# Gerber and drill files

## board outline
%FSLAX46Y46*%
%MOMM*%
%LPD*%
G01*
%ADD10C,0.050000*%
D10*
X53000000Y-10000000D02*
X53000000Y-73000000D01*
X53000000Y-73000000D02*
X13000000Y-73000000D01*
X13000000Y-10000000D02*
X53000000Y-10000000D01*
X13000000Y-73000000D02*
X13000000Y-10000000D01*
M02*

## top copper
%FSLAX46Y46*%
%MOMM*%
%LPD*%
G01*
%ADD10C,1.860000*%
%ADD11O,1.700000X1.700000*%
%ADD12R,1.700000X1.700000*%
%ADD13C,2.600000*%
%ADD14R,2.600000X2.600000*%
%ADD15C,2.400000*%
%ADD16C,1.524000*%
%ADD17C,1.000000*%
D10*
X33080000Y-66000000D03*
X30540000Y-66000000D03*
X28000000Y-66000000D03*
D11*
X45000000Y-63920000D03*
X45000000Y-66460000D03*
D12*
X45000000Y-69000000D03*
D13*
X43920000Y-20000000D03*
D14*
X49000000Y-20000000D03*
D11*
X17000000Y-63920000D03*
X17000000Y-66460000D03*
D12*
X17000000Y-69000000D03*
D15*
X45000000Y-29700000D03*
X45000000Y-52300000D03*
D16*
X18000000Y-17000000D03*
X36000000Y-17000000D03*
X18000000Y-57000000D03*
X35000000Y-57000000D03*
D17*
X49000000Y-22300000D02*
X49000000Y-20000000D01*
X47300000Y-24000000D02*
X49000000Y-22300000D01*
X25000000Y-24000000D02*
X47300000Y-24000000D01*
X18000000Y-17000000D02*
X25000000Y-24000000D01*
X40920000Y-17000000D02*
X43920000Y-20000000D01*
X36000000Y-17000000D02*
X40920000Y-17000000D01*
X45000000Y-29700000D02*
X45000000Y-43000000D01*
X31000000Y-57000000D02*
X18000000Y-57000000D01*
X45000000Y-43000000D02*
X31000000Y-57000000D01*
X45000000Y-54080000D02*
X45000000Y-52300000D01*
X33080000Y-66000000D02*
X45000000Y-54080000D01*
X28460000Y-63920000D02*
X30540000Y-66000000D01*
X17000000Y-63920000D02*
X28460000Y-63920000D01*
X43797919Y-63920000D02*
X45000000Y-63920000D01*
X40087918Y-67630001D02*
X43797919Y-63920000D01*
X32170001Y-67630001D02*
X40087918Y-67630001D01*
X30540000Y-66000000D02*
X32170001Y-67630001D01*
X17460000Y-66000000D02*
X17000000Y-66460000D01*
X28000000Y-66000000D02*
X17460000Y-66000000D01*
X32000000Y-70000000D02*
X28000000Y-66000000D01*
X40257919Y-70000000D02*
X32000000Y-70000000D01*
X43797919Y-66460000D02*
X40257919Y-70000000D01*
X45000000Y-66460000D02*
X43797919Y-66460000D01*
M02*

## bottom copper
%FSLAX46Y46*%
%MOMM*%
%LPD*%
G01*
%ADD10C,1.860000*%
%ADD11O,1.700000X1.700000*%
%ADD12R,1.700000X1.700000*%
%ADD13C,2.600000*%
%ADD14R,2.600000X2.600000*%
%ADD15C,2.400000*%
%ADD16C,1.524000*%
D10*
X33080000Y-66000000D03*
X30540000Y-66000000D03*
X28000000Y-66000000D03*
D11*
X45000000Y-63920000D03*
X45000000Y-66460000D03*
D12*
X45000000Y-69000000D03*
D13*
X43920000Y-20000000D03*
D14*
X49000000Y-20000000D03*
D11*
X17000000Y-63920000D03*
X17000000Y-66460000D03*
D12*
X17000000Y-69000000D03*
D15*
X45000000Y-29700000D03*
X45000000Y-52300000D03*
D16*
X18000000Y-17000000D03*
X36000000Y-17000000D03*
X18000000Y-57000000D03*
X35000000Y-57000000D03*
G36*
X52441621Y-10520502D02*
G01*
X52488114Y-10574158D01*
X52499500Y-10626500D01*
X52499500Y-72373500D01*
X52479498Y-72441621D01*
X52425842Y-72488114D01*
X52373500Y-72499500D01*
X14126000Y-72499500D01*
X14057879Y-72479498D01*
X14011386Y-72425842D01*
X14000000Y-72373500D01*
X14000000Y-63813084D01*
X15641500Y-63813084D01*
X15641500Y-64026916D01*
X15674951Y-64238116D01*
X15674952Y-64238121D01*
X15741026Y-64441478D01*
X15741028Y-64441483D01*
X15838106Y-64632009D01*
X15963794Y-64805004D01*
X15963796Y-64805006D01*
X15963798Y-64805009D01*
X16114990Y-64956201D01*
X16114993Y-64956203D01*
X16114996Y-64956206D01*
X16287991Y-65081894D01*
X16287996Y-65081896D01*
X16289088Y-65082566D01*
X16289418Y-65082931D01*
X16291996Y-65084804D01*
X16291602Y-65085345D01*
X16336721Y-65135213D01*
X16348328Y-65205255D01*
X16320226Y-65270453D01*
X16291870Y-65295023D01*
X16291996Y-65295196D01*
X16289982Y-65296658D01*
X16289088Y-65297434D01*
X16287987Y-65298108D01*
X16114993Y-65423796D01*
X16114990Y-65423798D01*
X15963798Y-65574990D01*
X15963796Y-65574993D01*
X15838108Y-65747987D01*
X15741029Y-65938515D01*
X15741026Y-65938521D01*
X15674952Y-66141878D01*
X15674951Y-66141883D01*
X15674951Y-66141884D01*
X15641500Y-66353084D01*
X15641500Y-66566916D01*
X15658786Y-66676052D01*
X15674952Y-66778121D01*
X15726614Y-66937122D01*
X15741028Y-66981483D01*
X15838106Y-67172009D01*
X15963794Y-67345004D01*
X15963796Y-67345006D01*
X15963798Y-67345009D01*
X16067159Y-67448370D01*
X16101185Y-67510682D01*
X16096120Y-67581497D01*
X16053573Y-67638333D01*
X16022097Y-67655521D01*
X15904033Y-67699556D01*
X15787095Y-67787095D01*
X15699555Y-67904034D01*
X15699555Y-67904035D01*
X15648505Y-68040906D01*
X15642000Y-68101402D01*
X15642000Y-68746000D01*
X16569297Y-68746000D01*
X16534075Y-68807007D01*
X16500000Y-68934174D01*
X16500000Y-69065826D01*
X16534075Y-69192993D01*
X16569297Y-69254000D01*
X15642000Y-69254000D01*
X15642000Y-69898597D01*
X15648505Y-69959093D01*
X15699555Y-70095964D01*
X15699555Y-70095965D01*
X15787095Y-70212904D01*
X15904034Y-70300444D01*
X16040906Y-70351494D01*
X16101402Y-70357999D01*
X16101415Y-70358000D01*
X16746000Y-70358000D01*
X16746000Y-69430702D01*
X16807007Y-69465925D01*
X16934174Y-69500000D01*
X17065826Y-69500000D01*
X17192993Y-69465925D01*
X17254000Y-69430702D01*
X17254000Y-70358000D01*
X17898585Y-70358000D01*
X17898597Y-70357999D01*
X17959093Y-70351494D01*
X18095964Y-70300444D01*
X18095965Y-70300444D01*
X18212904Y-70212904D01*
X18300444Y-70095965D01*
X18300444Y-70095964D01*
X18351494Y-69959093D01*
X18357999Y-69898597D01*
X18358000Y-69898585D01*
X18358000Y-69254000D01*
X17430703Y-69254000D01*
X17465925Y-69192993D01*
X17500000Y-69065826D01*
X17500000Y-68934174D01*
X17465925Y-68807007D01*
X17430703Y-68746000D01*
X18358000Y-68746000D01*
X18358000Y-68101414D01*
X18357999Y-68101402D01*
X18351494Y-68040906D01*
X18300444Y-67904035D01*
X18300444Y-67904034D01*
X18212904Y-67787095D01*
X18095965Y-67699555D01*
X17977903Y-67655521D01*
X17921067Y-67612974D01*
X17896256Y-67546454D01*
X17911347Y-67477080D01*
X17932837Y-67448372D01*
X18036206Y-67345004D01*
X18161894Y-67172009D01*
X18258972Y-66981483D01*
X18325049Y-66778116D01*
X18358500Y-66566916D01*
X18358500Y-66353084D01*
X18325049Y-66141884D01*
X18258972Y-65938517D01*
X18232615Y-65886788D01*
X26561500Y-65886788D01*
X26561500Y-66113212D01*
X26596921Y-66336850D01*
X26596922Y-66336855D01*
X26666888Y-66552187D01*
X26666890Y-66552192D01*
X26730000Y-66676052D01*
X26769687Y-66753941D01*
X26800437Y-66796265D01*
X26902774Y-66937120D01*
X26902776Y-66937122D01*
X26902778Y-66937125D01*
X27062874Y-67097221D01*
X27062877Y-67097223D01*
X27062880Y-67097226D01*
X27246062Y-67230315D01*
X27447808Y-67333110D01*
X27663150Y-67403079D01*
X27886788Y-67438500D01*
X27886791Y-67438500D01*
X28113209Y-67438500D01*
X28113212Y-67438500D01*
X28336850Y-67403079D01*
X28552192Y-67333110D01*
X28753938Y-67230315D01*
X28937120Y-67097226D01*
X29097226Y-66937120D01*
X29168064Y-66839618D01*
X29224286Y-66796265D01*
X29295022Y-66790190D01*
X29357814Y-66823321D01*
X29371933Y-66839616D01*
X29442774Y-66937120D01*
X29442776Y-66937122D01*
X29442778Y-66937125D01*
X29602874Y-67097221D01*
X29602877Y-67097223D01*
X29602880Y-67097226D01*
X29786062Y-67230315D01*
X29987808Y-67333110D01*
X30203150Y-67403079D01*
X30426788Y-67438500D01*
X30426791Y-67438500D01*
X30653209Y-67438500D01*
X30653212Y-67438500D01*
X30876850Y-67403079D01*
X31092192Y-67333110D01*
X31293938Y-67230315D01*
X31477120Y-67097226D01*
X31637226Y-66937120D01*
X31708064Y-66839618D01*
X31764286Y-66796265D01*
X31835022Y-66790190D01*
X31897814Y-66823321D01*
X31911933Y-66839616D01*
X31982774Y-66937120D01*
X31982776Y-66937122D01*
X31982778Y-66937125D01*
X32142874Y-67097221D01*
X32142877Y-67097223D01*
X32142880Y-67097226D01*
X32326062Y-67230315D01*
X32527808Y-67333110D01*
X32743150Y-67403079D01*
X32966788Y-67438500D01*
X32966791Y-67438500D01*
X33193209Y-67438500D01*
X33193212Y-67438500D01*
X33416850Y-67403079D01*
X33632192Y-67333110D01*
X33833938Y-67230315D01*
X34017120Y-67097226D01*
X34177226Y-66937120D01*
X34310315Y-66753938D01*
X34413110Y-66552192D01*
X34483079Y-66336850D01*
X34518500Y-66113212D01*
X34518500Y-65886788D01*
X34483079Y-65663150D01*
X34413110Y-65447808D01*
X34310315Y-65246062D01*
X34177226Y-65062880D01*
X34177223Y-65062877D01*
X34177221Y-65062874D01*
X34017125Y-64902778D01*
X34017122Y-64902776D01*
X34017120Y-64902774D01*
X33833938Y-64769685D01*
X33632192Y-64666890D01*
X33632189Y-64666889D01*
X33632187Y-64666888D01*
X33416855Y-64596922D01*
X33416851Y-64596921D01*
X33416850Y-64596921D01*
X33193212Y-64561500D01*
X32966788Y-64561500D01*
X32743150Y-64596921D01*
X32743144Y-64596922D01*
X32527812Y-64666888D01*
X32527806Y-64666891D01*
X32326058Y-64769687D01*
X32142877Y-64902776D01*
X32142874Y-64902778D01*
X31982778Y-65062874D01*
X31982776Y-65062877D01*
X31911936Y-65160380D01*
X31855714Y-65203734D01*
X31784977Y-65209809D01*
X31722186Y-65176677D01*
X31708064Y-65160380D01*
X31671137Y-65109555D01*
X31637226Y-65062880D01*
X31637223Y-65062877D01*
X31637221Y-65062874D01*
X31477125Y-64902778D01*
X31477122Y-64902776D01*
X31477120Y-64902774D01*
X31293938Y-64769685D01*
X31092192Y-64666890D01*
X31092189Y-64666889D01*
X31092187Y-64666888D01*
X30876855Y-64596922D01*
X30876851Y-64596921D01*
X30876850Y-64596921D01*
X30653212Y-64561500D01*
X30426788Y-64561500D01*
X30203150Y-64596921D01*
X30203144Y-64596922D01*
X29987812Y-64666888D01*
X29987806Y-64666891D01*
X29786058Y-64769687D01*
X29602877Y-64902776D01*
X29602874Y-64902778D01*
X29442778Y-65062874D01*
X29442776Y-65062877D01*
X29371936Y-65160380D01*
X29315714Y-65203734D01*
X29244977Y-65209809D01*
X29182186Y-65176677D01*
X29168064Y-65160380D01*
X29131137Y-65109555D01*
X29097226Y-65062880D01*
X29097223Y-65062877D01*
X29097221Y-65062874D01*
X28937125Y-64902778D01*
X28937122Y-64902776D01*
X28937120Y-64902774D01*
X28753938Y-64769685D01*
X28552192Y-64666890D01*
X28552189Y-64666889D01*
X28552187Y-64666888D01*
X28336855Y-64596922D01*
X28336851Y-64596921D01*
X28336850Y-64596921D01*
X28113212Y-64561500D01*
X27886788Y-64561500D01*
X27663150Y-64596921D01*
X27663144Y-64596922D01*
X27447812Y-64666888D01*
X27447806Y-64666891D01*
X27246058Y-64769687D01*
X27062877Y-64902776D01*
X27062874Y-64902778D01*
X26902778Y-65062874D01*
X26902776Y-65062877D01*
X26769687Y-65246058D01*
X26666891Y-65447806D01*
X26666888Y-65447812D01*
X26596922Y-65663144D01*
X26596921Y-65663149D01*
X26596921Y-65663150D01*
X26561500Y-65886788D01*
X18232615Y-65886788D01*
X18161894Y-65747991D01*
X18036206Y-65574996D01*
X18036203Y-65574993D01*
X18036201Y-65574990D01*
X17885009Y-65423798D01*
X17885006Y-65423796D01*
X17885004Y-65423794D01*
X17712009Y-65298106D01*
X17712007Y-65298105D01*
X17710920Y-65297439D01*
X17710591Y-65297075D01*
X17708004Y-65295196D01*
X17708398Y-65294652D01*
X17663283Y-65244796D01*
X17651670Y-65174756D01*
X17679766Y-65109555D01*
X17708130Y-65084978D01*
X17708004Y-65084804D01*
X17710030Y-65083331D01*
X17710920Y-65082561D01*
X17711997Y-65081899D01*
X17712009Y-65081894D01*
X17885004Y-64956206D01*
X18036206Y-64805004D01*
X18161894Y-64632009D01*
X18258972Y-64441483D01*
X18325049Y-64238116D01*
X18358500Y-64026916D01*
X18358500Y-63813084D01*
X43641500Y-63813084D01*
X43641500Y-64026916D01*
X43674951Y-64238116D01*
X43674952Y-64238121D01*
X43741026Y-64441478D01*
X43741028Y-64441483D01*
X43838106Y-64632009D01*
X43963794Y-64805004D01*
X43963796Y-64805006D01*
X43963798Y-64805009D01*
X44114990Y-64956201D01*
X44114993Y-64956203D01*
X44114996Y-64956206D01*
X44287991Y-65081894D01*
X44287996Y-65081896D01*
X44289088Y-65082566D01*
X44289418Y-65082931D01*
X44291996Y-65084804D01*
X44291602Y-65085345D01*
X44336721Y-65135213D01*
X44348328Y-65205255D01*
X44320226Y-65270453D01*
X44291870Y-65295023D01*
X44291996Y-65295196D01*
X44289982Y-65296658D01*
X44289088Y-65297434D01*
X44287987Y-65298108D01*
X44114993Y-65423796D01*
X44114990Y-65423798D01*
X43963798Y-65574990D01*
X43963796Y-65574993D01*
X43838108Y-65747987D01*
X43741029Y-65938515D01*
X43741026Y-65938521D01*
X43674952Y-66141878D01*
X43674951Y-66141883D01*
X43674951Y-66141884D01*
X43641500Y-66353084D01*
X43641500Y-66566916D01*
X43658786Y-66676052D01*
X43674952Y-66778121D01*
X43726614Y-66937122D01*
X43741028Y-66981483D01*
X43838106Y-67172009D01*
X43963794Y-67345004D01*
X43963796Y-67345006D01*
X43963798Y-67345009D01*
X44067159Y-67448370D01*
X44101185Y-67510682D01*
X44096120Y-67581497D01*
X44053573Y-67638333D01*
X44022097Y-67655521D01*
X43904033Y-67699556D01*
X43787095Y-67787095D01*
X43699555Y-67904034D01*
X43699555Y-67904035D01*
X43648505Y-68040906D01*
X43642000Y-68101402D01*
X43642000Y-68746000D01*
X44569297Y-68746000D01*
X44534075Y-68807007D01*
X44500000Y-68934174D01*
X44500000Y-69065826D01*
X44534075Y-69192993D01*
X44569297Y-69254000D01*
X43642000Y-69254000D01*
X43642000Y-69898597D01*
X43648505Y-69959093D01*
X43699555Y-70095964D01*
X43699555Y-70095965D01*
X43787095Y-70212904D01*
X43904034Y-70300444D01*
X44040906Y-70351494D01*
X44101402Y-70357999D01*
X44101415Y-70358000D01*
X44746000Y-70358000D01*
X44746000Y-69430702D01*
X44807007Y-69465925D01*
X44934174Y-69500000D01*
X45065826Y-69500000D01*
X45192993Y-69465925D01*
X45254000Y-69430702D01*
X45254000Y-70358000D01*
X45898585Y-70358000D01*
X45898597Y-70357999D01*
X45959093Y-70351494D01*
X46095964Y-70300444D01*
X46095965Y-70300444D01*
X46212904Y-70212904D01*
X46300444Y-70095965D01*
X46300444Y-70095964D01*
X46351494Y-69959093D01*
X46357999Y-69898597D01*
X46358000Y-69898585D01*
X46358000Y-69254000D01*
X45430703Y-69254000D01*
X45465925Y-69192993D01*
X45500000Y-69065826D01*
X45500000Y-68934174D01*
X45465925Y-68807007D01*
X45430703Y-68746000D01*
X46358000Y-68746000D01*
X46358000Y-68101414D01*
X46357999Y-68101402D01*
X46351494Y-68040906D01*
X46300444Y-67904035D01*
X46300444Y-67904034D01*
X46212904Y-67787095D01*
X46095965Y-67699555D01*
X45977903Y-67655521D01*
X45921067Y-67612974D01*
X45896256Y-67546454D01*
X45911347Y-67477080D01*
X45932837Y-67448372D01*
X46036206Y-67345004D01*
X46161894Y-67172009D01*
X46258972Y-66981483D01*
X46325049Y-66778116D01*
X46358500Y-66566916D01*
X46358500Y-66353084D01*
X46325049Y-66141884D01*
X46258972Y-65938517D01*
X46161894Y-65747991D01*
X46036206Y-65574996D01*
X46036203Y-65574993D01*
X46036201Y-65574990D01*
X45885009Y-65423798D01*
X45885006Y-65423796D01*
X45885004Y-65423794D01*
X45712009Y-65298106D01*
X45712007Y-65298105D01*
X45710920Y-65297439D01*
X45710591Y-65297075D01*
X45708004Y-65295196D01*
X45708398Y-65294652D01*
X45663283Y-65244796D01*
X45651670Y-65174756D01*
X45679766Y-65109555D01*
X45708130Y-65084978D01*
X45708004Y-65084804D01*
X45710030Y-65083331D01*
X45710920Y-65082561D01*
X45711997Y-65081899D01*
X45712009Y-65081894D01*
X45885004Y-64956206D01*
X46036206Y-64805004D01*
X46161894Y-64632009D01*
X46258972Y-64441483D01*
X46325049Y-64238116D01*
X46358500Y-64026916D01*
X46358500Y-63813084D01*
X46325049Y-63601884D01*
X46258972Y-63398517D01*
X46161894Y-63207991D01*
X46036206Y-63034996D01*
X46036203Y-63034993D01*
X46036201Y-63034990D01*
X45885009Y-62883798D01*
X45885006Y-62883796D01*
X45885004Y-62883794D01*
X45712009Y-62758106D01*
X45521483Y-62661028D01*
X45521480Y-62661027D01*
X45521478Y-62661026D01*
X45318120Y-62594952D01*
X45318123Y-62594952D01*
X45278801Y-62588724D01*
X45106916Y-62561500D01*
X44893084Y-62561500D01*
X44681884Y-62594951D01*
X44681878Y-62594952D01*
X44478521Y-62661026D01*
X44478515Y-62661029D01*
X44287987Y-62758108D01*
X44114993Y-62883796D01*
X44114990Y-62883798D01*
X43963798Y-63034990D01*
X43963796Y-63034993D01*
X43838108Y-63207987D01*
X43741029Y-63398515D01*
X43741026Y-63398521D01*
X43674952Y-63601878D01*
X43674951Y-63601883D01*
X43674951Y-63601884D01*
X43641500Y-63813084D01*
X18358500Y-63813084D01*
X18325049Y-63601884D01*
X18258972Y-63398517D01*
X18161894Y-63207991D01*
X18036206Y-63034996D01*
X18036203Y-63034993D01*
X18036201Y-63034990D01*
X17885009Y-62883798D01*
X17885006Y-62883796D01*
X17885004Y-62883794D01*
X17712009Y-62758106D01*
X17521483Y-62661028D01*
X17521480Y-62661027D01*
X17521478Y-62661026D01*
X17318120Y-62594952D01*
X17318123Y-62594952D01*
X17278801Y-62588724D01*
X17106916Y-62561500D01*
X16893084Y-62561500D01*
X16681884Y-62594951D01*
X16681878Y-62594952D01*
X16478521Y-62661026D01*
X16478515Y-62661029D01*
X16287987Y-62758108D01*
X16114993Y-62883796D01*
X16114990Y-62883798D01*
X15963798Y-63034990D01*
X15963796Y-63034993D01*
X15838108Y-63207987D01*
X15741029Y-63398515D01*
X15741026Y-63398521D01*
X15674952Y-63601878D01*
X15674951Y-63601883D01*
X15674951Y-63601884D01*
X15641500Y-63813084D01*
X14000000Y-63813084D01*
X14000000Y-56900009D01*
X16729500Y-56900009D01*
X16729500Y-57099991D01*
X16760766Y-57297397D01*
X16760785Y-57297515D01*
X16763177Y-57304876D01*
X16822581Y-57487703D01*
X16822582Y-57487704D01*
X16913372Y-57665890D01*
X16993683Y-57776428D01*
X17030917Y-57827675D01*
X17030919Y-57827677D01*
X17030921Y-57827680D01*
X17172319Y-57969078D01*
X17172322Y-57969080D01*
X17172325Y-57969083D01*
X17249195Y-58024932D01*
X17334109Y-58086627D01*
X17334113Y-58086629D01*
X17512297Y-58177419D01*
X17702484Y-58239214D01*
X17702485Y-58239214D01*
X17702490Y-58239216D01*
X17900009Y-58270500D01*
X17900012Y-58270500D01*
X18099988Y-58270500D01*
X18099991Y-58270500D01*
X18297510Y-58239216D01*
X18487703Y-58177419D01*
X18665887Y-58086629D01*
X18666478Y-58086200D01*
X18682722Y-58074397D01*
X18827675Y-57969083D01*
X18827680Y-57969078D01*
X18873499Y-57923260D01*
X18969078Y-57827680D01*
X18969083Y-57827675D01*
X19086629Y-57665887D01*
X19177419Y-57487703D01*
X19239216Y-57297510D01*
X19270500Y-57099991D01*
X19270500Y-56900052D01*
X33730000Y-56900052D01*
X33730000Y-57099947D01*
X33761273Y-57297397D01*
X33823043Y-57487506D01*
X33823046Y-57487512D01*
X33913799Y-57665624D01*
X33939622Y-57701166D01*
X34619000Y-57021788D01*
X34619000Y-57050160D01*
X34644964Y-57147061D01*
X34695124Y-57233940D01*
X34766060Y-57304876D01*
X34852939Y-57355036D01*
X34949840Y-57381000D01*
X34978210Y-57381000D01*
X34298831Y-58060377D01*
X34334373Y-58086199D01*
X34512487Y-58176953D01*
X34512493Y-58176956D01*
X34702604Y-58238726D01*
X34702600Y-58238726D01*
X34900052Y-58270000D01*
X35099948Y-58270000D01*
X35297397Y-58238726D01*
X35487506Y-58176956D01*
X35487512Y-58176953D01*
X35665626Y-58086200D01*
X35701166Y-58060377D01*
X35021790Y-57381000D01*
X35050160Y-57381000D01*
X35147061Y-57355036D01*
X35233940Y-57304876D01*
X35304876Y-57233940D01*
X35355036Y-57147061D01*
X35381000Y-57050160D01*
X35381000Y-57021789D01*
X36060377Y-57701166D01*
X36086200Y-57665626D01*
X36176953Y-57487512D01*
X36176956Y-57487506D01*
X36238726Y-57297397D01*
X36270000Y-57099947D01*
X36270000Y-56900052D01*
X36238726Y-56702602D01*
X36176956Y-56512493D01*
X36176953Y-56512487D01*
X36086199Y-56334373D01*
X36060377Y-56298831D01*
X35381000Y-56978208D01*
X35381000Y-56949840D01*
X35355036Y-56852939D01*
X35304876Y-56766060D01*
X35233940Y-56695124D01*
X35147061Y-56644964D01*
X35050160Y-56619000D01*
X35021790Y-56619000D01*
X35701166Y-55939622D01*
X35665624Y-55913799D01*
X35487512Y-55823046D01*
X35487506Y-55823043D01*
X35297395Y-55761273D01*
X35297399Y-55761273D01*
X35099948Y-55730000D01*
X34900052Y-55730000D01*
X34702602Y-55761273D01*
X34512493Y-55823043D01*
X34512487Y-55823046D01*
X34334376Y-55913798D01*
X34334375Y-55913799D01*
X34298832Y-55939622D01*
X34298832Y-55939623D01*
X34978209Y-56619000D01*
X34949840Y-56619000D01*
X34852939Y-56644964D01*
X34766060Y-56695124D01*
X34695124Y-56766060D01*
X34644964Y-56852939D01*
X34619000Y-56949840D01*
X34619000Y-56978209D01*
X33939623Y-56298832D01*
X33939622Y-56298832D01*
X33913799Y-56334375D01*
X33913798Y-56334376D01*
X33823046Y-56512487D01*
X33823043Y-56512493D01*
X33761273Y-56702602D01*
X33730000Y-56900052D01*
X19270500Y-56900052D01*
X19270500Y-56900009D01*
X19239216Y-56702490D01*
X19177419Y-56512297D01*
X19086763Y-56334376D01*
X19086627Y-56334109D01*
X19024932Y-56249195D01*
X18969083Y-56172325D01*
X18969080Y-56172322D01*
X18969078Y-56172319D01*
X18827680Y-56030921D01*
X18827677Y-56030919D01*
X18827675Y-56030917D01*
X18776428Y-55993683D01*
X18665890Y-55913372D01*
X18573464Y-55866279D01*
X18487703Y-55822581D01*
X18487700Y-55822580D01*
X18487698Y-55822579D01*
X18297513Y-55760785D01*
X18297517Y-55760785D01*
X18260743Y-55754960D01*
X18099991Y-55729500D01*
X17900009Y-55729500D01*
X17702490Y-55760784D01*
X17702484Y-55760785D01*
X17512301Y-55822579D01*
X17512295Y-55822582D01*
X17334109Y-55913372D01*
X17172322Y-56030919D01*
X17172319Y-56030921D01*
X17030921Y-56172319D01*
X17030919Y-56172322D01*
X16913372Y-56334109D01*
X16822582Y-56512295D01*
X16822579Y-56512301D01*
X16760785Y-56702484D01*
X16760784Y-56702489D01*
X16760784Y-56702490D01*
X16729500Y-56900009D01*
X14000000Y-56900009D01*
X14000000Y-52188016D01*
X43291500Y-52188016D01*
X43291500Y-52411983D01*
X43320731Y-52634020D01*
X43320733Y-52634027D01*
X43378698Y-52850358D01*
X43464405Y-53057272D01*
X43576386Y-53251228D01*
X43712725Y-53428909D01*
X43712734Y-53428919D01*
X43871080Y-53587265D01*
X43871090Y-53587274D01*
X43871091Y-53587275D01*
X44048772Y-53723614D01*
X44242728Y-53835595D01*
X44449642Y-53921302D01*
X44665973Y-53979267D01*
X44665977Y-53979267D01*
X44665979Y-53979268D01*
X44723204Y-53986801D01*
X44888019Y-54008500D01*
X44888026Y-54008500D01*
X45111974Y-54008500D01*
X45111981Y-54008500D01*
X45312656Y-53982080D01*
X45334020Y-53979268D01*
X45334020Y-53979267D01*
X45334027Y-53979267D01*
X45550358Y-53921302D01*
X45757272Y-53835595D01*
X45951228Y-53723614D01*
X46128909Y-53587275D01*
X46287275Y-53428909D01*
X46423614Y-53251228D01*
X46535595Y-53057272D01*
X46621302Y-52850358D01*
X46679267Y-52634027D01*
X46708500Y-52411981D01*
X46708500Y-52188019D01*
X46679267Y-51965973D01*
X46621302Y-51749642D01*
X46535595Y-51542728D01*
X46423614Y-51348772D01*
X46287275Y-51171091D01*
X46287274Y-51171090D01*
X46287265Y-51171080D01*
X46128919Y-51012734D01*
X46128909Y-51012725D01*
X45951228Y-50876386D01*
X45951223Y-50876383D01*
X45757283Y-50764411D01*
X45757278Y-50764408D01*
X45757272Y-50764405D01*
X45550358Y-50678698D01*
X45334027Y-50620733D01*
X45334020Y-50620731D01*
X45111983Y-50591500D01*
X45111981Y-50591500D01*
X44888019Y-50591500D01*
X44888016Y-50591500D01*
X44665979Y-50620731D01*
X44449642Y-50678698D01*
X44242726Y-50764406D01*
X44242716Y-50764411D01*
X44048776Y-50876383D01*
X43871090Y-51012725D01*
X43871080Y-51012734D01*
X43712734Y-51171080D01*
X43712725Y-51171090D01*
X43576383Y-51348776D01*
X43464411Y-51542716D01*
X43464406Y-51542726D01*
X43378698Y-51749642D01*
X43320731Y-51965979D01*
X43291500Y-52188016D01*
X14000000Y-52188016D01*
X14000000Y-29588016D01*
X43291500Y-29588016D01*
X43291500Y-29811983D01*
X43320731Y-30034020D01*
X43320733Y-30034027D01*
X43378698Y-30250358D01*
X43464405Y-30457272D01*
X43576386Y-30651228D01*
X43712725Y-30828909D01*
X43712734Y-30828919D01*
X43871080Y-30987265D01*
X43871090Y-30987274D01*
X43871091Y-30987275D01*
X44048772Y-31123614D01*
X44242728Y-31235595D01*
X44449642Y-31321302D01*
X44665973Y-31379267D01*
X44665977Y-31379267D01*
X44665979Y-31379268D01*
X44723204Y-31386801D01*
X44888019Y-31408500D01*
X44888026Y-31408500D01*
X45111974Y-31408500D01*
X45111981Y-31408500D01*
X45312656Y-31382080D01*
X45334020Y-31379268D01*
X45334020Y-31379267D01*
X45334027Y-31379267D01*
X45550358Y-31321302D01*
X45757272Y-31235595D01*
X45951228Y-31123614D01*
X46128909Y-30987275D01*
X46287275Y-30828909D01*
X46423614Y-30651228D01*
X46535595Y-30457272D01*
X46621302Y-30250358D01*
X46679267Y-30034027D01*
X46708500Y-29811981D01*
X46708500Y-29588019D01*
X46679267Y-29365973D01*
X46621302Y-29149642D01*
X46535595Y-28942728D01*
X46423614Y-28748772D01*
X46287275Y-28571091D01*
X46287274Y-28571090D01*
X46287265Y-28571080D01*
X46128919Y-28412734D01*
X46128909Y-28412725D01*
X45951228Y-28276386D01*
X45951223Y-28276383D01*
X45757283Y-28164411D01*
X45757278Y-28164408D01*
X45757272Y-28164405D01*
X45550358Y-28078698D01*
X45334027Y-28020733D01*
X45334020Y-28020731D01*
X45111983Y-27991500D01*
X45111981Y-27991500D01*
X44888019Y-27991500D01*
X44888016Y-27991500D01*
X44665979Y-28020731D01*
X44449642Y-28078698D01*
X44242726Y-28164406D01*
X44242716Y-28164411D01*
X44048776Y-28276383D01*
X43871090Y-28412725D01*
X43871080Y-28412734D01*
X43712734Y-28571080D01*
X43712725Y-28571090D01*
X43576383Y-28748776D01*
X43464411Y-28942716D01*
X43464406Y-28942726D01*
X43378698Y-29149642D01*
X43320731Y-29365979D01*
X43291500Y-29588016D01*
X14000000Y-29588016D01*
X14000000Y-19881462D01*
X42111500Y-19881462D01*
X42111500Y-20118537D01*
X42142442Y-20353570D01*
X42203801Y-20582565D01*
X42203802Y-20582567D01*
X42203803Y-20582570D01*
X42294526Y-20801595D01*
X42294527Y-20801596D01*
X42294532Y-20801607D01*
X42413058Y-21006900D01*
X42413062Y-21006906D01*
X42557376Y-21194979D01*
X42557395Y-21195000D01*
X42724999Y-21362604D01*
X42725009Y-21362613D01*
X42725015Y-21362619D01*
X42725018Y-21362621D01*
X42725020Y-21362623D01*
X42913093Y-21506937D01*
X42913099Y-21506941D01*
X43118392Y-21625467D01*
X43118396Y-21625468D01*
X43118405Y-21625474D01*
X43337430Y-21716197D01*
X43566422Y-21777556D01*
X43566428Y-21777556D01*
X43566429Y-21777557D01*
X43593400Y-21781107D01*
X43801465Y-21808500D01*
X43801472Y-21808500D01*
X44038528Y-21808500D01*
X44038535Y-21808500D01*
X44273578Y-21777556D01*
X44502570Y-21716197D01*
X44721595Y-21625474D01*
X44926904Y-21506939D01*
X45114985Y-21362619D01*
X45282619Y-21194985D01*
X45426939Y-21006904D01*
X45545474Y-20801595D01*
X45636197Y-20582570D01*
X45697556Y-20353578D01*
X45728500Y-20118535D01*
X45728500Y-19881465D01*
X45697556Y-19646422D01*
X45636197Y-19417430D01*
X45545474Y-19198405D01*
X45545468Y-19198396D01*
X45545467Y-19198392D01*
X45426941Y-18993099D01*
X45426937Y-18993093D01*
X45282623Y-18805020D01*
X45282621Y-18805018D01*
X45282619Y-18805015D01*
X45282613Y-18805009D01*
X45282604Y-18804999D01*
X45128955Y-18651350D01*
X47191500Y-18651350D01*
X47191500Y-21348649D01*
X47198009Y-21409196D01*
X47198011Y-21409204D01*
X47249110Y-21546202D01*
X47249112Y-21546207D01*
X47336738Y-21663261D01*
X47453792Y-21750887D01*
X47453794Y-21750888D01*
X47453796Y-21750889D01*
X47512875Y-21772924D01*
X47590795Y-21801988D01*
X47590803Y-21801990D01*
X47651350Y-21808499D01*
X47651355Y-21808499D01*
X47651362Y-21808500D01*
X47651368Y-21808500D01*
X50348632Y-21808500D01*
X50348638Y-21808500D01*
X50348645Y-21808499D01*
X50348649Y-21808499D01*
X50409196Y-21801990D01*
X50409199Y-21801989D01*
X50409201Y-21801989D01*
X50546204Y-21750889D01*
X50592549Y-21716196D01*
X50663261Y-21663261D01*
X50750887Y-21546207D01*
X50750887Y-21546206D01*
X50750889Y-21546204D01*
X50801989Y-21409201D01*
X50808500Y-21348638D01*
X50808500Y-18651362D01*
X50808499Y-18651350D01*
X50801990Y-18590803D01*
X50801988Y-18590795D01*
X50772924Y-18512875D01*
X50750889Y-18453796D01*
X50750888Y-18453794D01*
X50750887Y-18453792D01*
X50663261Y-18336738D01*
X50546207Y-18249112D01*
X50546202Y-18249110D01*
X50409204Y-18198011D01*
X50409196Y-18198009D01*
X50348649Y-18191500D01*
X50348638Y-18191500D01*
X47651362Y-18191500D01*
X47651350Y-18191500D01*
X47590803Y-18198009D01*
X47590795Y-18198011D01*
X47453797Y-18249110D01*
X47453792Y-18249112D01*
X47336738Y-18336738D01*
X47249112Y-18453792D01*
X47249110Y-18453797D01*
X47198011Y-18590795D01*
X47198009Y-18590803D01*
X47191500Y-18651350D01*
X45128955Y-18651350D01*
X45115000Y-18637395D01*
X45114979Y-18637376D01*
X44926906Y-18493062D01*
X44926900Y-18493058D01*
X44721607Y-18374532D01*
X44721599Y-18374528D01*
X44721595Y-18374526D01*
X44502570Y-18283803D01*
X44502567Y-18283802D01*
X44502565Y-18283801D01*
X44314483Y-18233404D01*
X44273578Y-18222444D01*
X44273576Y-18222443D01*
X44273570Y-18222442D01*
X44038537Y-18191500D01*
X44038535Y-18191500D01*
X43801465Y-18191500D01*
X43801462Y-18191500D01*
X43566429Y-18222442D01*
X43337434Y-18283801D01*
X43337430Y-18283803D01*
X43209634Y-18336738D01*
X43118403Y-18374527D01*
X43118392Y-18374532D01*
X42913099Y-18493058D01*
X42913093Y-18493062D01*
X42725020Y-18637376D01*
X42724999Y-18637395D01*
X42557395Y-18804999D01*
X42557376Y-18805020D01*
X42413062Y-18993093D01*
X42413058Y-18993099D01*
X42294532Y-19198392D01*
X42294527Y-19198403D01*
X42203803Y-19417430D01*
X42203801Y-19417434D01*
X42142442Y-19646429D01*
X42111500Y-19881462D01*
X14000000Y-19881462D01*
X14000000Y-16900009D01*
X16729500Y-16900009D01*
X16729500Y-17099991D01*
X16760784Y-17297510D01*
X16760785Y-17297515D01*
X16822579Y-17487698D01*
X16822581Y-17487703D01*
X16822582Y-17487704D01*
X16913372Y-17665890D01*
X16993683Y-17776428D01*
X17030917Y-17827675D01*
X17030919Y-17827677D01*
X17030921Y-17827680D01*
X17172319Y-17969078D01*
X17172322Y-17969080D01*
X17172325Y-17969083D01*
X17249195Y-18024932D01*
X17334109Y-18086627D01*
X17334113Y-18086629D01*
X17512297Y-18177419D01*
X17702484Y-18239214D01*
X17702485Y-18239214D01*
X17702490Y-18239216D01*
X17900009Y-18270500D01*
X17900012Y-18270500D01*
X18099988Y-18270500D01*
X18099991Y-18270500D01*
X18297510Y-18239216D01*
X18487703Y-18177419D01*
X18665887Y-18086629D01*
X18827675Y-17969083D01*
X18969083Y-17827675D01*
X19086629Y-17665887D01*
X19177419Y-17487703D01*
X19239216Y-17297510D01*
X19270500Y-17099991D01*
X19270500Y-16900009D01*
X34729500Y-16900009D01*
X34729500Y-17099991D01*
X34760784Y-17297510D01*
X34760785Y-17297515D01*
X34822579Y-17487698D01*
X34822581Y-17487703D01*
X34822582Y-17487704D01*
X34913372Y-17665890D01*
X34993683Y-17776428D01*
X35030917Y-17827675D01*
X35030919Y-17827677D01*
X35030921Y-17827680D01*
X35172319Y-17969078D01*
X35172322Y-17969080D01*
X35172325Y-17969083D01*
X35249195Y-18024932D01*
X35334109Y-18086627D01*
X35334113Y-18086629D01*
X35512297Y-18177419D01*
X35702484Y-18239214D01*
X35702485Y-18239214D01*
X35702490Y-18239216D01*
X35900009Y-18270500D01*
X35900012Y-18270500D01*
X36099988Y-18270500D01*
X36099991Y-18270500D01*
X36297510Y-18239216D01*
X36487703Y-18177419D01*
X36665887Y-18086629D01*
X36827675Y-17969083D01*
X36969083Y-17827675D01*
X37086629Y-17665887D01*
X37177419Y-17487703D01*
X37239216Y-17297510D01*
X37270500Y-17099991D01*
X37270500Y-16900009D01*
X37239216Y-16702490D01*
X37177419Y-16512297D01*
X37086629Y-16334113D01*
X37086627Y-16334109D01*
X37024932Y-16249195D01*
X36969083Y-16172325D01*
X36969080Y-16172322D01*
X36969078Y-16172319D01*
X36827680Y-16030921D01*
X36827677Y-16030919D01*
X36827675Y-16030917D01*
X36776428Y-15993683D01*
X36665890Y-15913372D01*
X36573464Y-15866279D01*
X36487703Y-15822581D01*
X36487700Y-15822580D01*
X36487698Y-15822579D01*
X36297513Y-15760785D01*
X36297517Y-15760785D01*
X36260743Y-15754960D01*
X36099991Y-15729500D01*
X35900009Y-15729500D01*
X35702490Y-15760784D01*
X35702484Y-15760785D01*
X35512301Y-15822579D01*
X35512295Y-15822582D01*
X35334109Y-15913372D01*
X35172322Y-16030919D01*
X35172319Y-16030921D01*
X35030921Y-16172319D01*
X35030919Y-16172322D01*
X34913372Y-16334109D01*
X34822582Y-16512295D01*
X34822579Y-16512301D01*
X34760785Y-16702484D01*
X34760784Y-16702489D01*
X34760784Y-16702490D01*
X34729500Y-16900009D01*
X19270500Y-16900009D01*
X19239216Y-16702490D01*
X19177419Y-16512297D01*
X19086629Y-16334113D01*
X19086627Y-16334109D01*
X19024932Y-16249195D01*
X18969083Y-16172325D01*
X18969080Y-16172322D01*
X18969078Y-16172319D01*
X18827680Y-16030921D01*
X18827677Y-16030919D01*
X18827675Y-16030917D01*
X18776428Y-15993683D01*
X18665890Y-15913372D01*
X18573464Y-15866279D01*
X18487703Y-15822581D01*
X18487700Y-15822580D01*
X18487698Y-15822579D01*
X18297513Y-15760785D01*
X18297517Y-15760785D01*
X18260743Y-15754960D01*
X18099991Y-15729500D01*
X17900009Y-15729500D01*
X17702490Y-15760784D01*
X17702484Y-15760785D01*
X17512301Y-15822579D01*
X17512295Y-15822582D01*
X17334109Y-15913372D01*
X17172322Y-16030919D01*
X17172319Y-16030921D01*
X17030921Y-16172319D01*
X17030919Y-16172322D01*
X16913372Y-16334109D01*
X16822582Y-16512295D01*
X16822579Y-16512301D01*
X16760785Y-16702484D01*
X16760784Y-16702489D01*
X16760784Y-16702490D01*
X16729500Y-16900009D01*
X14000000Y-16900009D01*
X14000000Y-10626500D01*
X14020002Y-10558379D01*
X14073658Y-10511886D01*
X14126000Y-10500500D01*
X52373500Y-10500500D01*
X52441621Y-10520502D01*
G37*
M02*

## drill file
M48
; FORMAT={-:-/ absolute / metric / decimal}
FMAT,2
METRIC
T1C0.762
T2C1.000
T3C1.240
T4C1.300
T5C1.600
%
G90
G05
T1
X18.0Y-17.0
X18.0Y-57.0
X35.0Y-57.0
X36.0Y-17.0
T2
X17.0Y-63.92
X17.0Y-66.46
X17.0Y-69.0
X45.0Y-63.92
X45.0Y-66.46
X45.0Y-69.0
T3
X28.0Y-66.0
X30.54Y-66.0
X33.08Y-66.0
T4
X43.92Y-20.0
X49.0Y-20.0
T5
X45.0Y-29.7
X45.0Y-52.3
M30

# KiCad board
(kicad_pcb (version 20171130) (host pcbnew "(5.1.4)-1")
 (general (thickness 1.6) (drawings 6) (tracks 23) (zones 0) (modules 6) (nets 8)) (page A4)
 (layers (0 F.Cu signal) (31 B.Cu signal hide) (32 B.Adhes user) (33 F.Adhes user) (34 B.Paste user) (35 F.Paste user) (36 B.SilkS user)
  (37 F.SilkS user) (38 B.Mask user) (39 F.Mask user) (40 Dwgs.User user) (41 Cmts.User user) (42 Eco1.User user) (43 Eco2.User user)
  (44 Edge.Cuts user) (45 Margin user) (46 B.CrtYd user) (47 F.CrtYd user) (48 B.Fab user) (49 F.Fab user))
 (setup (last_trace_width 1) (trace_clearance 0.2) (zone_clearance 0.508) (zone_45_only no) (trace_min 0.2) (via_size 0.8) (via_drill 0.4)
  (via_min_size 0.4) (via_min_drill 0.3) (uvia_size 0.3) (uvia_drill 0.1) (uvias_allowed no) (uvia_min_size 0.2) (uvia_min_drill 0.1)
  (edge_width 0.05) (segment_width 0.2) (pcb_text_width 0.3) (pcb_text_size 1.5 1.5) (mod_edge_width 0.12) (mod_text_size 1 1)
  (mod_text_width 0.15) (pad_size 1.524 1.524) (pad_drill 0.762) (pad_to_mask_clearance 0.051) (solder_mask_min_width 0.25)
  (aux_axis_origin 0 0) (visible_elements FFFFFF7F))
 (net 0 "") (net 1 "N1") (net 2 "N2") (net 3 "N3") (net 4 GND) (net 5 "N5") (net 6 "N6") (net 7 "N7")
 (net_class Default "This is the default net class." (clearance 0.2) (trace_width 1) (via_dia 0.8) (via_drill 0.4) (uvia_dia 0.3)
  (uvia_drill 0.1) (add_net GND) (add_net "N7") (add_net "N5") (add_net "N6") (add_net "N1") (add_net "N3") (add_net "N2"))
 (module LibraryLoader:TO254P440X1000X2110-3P (layer F.Cu) (at 28 66)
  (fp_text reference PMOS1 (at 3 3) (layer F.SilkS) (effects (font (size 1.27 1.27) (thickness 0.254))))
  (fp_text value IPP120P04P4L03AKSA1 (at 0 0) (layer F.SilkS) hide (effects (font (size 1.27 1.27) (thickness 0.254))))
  (pad 3 thru_hole circle (at 5.08 0) (size 1.86 1.86) (drill 1.24) (layers *.Cu *.Mask) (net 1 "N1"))
  (pad 2 thru_hole circle (at 2.54 0) (size 1.86 1.86) (drill 1.24) (layers *.Cu *.Mask) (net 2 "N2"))
  (pad 1 thru_hole circle (at 0 0) (size 1.86 1.86) (drill 1.24) (layers *.Cu *.Mask) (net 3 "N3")))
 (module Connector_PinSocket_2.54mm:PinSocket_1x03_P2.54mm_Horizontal (layer F.Cu) (at 45 69 180)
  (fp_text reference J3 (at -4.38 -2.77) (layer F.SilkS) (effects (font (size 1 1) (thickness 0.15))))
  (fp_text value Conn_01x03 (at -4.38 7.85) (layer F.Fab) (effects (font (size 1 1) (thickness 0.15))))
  (pad 3 thru_hole oval (at 0 5.08 180) (size 1.7 1.7) (drill 1) (layers *.Cu *.Mask) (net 2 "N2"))
  (pad 2 thru_hole oval (at 0 2.54 180) (size 1.7 1.7) (drill 1) (layers *.Cu *.Mask) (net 3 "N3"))
  (pad 1 thru_hole rect (at 0 0 180) (size 1.7 1.7) (drill 1) (layers *.Cu *.Mask) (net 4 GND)))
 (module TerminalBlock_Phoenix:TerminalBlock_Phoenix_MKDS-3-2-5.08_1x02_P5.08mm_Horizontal (layer F.Cu) (at 49 20 180)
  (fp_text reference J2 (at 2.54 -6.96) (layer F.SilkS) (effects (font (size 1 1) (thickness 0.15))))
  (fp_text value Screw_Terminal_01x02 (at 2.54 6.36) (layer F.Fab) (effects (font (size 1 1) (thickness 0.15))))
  (pad 2 thru_hole circle (at 5.08 0 180) (size 2.6 2.6) (drill 1.3) (layers *.Cu *.Mask) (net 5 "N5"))
  (pad 1 thru_hole rect (at 0 0 180) (size 2.6 2.6) (drill 1.3) (layers *.Cu *.Mask) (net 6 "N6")))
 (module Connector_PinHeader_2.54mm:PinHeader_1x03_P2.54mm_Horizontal (layer F.Cu) (at 17 69 180)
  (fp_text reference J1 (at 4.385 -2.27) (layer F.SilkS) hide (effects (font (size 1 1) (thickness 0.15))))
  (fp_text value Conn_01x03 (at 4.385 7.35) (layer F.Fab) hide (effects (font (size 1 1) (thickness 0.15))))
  (pad 3 thru_hole oval (at 0 5.08 180) (size 1.7 1.7) (drill 1) (layers *.Cu *.Mask) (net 2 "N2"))
  (pad 2 thru_hole oval (at 0 2.54 180) (size 1.7 1.7) (drill 1) (layers *.Cu *.Mask) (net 3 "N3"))
  (pad 1 thru_hole rect (at 0 0 180) (size 1.7 1.7) (drill 1) (layers *.Cu *.Mask) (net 4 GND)))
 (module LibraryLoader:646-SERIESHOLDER (layer F.Cu) (at 45 41 90)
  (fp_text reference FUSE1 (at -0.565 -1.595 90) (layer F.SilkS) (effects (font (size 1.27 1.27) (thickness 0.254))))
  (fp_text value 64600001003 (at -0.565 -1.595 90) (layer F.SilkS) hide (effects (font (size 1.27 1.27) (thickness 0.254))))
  (pad 2 thru_hole circle (at 11.3 0 90) (size 2.4 2.4) (drill 1.6) (layers *.Cu *.Mask) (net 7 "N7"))
  (pad 1 thru_hole circle (at -11.3 0 90) (size 2.4 2.4) (drill 1.6) (layers *.Cu *.Mask) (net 1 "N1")))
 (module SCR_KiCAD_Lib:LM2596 (layer F.Cu) (at 25 60 180)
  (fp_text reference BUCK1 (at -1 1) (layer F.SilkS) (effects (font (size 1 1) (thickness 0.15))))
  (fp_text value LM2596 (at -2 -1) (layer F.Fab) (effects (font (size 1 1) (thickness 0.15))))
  (pad 4 thru_hole circle (at 7 43 180) (size 1.524 1.524) (drill 0.762) (layers *.Cu *.Mask) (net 6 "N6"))
  (pad 3 thru_hole circle (at -11 43 180) (size 1.524 1.524) (drill 0.762) (layers *.Cu *.Mask) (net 5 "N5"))
  (pad 2 thru_hole circle (at 7 3 180) (size 1.524 1.524) (drill 0.762) (layers *.Cu *.Mask) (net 7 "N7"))
  (pad 1 thru_hole circle (at -10 3 180) (size 1.524 1.524) (drill 0.762) (layers *.Cu *.Mask) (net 4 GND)))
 (gr_line (start 53 10) (end 53 73) (layer Edge.Cuts) (width 0.05))
 (gr_line (start 53 73) (end 13 73) (layer Edge.Cuts) (width 0.05))
 (gr_line (start 13 10) (end 53 10) (layer Edge.Cuts) (width 0.05))
 (gr_line (start 13 73) (end 13 10) (layer Edge.Cuts) (width 0.05))
 (segment (start 49 22.3) (end 49 20) (width 1) (layer F.Cu) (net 6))
 (segment (start 47.3 24) (end 49 22.3) (width 1) (layer F.Cu) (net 6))
 (segment (start 25 24) (end 47.3 24) (width 1) (layer F.Cu) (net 6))
 (segment (start 18 17) (end 25 24) (width 1) (layer F.Cu) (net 6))
 (segment (start 40.92 17) (end 43.92 20) (width 1) (layer F.Cu) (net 5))
 (segment (start 36 17) (end 40.92 17) (width 1) (layer F.Cu) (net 5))
 (segment (start 45 29.7) (end 45 43) (width 1) (layer F.Cu) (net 7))
 (segment (start 31 57) (end 18 57) (width 1) (layer F.Cu) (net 7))
 (segment (start 45 43) (end 31 57) (width 1) (layer F.Cu) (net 7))
 (segment (start 45 54.08) (end 45 52.3) (width 1) (layer F.Cu) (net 1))
 (segment (start 33.08 66) (end 45 54.08) (width 1) (layer F.Cu) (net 1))
 (segment (start 28.46 63.92) (end 30.54 66) (width 1) (layer F.Cu) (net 2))
 (segment (start 17 63.92) (end 28.46 63.92) (width 1) (layer F.Cu) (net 2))
 (segment (start 43.797919 63.92) (end 45 63.92) (width 1) (layer F.Cu) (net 2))
 (segment (start 40.087918 67.630001) (end 43.797919 63.92) (width 1) (layer F.Cu) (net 2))
 (segment (start 32.170001 67.630001) (end 40.087918 67.630001) (width 1) (layer F.Cu) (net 2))
 (segment (start 30.54 66) (end 32.170001 67.630001) (width 1) (layer F.Cu) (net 2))
 (segment (start 17.46 66) (end 17 66.46) (width 1) (layer F.Cu) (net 3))
 (segment (start 28 66) (end 17.46 66) (width 1) (layer F.Cu) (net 3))
 (segment (start 32 70) (end 28 66) (width 1) (layer F.Cu) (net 3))
 (segment (start 40.257919 70) (end 32 70) (width 1) (layer F.Cu) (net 3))
 (segment (start 43.797919 66.46) (end 40.257919 70) (width 1) (layer F.Cu) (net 3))
 (segment (start 45 66.46) (end 43.797919 66.46) (width 1) (layer F.Cu) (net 3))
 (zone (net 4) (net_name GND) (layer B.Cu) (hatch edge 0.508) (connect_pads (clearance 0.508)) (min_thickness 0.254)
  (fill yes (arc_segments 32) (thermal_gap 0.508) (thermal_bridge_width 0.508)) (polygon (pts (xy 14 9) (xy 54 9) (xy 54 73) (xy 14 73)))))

